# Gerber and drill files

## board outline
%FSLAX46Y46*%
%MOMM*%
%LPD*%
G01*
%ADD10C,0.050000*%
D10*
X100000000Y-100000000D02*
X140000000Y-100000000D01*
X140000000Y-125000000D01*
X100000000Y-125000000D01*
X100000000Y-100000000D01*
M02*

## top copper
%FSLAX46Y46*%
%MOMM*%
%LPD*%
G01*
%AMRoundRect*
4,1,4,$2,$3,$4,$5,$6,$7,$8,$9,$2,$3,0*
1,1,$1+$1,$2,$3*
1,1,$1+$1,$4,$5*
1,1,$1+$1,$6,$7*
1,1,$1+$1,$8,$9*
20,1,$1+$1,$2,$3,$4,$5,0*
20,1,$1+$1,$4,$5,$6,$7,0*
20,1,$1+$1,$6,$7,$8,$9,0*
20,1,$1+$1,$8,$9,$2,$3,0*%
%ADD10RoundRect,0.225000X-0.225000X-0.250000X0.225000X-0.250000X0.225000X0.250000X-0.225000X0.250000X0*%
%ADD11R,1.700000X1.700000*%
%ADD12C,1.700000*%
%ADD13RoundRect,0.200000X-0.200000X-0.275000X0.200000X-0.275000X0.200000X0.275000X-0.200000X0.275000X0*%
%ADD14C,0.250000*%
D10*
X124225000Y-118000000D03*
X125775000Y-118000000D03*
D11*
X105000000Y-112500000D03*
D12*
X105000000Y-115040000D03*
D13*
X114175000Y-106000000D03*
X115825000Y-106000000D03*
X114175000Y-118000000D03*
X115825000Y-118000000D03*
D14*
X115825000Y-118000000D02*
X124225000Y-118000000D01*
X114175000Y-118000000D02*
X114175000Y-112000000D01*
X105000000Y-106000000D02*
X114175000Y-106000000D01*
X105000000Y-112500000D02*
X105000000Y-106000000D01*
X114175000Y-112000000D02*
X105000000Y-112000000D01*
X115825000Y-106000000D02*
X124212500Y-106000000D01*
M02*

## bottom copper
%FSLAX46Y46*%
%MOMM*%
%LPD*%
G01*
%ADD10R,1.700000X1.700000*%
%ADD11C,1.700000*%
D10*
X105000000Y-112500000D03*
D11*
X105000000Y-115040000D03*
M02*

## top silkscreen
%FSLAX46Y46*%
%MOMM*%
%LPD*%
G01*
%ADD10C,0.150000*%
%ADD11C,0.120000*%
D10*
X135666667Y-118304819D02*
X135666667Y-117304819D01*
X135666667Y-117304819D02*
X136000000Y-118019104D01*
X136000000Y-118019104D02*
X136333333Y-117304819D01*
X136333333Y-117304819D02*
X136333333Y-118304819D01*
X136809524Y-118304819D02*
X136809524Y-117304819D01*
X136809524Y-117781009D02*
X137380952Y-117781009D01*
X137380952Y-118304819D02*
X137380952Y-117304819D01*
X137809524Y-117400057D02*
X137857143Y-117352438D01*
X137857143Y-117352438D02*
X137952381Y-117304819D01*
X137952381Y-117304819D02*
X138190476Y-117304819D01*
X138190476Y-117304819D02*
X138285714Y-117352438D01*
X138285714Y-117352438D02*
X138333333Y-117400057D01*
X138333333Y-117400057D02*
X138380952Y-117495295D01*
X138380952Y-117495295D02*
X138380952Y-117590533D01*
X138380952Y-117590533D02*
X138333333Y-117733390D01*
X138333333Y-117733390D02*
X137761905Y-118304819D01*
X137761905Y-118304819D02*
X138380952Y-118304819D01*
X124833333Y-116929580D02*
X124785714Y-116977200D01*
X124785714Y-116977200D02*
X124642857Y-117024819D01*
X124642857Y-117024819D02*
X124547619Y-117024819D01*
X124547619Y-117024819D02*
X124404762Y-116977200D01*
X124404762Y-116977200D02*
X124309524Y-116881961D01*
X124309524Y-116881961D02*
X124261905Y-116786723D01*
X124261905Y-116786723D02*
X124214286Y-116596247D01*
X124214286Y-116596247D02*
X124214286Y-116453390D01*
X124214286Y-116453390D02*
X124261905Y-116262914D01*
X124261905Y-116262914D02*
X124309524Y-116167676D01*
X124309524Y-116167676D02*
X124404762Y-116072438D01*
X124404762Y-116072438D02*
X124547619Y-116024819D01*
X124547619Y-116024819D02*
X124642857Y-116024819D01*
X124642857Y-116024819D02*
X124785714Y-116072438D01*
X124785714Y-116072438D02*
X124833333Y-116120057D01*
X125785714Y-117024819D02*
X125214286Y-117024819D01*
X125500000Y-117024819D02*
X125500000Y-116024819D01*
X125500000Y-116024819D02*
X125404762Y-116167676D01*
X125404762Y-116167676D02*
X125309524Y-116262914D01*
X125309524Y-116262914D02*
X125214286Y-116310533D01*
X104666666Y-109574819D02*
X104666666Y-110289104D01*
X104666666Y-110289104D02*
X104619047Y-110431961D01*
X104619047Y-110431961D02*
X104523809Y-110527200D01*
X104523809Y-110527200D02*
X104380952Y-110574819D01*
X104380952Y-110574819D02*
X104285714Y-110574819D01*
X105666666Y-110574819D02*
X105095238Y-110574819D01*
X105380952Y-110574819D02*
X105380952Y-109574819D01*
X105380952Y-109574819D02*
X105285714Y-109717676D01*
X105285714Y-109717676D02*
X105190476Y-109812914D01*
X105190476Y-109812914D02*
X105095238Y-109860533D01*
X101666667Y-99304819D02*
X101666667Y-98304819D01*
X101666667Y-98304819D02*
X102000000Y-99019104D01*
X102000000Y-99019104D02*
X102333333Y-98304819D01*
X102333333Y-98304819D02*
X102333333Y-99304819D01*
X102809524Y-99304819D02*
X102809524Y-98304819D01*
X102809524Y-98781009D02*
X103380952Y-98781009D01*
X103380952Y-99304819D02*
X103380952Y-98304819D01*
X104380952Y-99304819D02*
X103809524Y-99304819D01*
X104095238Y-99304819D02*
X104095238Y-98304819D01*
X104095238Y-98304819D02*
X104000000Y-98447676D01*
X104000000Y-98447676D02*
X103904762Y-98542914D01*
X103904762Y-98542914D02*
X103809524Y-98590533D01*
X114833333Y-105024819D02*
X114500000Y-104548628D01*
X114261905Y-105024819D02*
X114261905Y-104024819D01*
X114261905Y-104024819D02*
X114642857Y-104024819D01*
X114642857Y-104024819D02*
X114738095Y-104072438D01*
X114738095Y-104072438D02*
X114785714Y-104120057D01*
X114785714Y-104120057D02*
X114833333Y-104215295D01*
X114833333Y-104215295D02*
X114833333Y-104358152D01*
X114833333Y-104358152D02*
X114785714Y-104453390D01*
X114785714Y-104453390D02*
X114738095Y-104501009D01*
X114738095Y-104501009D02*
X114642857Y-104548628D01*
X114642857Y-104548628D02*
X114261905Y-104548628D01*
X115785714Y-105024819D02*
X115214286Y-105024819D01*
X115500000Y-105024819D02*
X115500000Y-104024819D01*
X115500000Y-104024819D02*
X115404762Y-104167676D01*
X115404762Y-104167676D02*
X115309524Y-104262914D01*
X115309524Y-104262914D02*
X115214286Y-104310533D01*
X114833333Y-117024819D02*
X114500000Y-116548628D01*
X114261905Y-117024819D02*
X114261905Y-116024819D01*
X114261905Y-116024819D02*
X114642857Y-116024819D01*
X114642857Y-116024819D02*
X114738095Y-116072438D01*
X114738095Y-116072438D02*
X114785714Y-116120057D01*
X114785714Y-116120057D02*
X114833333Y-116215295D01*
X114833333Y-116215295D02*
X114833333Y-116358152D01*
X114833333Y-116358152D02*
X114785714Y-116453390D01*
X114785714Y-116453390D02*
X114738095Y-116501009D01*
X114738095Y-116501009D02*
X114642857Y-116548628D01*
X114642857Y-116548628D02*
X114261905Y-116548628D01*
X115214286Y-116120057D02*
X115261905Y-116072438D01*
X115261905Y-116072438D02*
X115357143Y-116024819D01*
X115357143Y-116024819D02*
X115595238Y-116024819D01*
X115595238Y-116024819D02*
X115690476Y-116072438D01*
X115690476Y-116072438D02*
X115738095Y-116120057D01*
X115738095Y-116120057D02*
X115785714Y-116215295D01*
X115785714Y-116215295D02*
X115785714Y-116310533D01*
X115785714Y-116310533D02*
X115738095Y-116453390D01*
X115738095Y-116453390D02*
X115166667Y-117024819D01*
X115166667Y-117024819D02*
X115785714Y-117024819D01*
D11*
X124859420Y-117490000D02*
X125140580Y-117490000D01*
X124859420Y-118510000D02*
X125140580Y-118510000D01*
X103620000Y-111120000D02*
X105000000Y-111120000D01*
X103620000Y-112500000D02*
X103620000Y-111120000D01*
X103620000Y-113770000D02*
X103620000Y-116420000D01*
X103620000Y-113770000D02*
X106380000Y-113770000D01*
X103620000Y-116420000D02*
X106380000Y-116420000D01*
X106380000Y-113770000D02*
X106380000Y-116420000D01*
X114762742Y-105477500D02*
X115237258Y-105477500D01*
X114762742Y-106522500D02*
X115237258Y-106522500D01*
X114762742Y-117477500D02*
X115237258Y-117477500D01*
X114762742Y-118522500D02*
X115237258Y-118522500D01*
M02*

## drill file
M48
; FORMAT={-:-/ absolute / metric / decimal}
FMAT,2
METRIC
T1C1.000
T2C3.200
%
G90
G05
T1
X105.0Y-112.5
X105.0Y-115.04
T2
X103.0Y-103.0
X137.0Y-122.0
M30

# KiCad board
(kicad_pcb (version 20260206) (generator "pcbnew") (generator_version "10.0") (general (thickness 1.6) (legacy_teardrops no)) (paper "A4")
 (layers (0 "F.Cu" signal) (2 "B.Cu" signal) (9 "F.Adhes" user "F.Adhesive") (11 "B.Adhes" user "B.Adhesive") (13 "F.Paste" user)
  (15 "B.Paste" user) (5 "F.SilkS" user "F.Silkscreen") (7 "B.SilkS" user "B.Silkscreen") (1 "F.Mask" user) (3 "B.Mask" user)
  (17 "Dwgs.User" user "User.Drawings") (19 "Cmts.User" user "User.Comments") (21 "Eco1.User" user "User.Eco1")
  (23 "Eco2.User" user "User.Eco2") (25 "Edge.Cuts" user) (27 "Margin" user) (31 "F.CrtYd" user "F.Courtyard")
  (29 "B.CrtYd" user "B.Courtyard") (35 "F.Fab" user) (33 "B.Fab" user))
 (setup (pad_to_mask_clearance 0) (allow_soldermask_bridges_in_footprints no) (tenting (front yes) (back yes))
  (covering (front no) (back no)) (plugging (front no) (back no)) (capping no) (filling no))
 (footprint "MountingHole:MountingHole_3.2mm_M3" (layer "F.Cu") (at 137 122)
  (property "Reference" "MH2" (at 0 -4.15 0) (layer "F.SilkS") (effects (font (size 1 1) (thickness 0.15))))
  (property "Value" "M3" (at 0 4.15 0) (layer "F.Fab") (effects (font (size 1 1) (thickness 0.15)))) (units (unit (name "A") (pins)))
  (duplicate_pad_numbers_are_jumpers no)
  (pad "" np_thru_hole circle (at 0 0) (size 3.2 3.2) (drill 3.2) (layers "*.Cu" "*.Mask")))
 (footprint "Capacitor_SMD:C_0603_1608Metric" (layer "F.Cu") (at 125 118)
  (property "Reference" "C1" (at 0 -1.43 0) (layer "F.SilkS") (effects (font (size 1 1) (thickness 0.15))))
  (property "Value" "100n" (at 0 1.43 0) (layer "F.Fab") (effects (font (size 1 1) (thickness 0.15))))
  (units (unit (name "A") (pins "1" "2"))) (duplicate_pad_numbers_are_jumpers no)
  (fp_line (start -0.14058 -0.51) (end 0.14058 -0.51) (stroke (width 0.12) (type solid)) (layer "F.SilkS"))
  (fp_line (start -0.14058 0.51) (end 0.14058 0.51) (stroke (width 0.12) (type solid)) (layer "F.SilkS"))
  (pad "1" smd roundrect (at -0.775 0) (size 0.9 0.95) (layers "F.Cu" "F.Mask" "F.Paste") (roundrect_rratio 0.25) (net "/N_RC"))
  (pad "2" smd roundrect (at 0.775 0) (size 0.9 0.95) (layers "F.Cu" "F.Mask" "F.Paste") (roundrect_rratio 0.25) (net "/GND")))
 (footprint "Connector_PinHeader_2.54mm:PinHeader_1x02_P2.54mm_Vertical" (layer "F.Cu") (at 105 112.5)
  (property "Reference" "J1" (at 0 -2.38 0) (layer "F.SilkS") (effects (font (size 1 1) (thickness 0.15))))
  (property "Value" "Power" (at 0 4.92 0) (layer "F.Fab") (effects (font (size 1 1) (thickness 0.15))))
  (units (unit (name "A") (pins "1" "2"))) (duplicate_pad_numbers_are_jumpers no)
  (fp_line (start -1.38 -1.38) (end 0 -1.38) (stroke (width 0.12) (type solid)) (layer "F.SilkS"))
  (fp_line (start -1.38 0) (end -1.38 -1.38) (stroke (width 0.12) (type solid)) (layer "F.SilkS"))
  (fp_line (start -1.38 1.27) (end -1.38 3.92) (stroke (width 0.12) (type solid)) (layer "F.SilkS"))
  (fp_line (start -1.38 1.27) (end 1.38 1.27) (stroke (width 0.12) (type solid)) (layer "F.SilkS"))
  (fp_line (start -1.38 3.92) (end 1.38 3.92) (stroke (width 0.12) (type solid)) (layer "F.SilkS"))
  (fp_line (start 1.38 1.27) (end 1.38 3.92) (stroke (width 0.12) (type solid)) (layer "F.SilkS"))
  (pad "1" thru_hole rect (at 0 0) (size 1.7 1.7) (drill 1) (layers "*.Cu" "*.Mask") (remove_unused_layers no) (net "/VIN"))
  (pad "2" thru_hole circle (at 0 2.54) (size 1.7 1.7) (drill 1) (layers "*.Cu" "*.Mask") (remove_unused_layers no) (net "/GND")))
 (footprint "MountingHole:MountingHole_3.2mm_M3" (layer "F.Cu") (at 103 103)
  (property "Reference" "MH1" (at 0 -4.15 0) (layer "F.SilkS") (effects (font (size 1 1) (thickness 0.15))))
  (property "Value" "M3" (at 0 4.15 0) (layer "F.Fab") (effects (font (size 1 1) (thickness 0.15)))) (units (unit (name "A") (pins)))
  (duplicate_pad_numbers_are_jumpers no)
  (pad "" np_thru_hole circle (at 0 0) (size 3.2 3.2) (drill 3.2) (layers "*.Cu" "*.Mask")))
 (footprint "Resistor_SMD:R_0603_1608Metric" (layer "F.Cu") (at 115 106)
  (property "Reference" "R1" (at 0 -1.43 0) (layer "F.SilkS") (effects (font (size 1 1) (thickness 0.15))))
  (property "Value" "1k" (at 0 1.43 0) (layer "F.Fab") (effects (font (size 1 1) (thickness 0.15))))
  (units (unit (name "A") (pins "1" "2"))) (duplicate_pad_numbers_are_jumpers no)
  (fp_line (start -0.237258 -0.5225) (end 0.237258 -0.5225) (stroke (width 0.12) (type solid)) (layer "F.SilkS"))
  (fp_line (start -0.237258 0.5225) (end 0.237258 0.5225) (stroke (width 0.12) (type solid)) (layer "F.SilkS"))
  (pad "1" smd roundrect (at -0.825 0) (size 0.8 0.95) (layers "F.Cu" "F.Mask" "F.Paste") (roundrect_rratio 0.25) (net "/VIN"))
  (pad "2" smd roundrect (at 0.825 0) (size 0.8 0.95) (layers "F.Cu" "F.Mask" "F.Paste") (roundrect_rratio 0.25) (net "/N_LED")))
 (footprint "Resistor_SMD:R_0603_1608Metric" (layer "F.Cu") (at 115 118)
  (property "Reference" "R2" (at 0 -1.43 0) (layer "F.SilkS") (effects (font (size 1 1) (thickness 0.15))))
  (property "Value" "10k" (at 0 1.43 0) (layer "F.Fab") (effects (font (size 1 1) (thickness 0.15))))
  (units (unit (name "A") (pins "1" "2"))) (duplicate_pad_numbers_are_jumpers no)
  (fp_line (start -0.237258 -0.5225) (end 0.237258 -0.5225) (stroke (width 0.12) (type solid)) (layer "F.SilkS"))
  (fp_line (start -0.237258 0.5225) (end 0.237258 0.5225) (stroke (width 0.12) (type solid)) (layer "F.SilkS"))
  (pad "1" smd roundrect (at -0.825 0) (size 0.8 0.95) (layers "F.Cu" "F.Mask" "F.Paste") (roundrect_rratio 0.25) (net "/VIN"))
  (pad "2" smd roundrect (at 0.825 0) (size 0.8 0.95) (layers "F.Cu" "F.Mask" "F.Paste") (roundrect_rratio 0.25) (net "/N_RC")))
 (gr_rect (start 100 100) (end 140 125) (stroke (width 0.05) (type default)) (fill no) (layer "Edge.Cuts"))
 (segment (start 115.825 118) (end 124.225 118) (width 0.25) (layer "F.Cu") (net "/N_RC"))
 (segment (start 114.175 118) (end 114.175 112) (width 0.25) (layer "F.Cu") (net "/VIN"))
 (segment (start 105 106) (end 114.175 106) (width 0.25) (layer "F.Cu") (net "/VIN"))
 (segment (start 105 112.5) (end 105 106) (width 0.25) (layer "F.Cu") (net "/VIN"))
 (segment (start 114.175 112) (end 105 112) (width 0.25) (layer "F.Cu") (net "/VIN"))
 (segment (start 115.825 106) (end 124.2125 106) (width 0.25) (layer "F.Cu") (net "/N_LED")))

